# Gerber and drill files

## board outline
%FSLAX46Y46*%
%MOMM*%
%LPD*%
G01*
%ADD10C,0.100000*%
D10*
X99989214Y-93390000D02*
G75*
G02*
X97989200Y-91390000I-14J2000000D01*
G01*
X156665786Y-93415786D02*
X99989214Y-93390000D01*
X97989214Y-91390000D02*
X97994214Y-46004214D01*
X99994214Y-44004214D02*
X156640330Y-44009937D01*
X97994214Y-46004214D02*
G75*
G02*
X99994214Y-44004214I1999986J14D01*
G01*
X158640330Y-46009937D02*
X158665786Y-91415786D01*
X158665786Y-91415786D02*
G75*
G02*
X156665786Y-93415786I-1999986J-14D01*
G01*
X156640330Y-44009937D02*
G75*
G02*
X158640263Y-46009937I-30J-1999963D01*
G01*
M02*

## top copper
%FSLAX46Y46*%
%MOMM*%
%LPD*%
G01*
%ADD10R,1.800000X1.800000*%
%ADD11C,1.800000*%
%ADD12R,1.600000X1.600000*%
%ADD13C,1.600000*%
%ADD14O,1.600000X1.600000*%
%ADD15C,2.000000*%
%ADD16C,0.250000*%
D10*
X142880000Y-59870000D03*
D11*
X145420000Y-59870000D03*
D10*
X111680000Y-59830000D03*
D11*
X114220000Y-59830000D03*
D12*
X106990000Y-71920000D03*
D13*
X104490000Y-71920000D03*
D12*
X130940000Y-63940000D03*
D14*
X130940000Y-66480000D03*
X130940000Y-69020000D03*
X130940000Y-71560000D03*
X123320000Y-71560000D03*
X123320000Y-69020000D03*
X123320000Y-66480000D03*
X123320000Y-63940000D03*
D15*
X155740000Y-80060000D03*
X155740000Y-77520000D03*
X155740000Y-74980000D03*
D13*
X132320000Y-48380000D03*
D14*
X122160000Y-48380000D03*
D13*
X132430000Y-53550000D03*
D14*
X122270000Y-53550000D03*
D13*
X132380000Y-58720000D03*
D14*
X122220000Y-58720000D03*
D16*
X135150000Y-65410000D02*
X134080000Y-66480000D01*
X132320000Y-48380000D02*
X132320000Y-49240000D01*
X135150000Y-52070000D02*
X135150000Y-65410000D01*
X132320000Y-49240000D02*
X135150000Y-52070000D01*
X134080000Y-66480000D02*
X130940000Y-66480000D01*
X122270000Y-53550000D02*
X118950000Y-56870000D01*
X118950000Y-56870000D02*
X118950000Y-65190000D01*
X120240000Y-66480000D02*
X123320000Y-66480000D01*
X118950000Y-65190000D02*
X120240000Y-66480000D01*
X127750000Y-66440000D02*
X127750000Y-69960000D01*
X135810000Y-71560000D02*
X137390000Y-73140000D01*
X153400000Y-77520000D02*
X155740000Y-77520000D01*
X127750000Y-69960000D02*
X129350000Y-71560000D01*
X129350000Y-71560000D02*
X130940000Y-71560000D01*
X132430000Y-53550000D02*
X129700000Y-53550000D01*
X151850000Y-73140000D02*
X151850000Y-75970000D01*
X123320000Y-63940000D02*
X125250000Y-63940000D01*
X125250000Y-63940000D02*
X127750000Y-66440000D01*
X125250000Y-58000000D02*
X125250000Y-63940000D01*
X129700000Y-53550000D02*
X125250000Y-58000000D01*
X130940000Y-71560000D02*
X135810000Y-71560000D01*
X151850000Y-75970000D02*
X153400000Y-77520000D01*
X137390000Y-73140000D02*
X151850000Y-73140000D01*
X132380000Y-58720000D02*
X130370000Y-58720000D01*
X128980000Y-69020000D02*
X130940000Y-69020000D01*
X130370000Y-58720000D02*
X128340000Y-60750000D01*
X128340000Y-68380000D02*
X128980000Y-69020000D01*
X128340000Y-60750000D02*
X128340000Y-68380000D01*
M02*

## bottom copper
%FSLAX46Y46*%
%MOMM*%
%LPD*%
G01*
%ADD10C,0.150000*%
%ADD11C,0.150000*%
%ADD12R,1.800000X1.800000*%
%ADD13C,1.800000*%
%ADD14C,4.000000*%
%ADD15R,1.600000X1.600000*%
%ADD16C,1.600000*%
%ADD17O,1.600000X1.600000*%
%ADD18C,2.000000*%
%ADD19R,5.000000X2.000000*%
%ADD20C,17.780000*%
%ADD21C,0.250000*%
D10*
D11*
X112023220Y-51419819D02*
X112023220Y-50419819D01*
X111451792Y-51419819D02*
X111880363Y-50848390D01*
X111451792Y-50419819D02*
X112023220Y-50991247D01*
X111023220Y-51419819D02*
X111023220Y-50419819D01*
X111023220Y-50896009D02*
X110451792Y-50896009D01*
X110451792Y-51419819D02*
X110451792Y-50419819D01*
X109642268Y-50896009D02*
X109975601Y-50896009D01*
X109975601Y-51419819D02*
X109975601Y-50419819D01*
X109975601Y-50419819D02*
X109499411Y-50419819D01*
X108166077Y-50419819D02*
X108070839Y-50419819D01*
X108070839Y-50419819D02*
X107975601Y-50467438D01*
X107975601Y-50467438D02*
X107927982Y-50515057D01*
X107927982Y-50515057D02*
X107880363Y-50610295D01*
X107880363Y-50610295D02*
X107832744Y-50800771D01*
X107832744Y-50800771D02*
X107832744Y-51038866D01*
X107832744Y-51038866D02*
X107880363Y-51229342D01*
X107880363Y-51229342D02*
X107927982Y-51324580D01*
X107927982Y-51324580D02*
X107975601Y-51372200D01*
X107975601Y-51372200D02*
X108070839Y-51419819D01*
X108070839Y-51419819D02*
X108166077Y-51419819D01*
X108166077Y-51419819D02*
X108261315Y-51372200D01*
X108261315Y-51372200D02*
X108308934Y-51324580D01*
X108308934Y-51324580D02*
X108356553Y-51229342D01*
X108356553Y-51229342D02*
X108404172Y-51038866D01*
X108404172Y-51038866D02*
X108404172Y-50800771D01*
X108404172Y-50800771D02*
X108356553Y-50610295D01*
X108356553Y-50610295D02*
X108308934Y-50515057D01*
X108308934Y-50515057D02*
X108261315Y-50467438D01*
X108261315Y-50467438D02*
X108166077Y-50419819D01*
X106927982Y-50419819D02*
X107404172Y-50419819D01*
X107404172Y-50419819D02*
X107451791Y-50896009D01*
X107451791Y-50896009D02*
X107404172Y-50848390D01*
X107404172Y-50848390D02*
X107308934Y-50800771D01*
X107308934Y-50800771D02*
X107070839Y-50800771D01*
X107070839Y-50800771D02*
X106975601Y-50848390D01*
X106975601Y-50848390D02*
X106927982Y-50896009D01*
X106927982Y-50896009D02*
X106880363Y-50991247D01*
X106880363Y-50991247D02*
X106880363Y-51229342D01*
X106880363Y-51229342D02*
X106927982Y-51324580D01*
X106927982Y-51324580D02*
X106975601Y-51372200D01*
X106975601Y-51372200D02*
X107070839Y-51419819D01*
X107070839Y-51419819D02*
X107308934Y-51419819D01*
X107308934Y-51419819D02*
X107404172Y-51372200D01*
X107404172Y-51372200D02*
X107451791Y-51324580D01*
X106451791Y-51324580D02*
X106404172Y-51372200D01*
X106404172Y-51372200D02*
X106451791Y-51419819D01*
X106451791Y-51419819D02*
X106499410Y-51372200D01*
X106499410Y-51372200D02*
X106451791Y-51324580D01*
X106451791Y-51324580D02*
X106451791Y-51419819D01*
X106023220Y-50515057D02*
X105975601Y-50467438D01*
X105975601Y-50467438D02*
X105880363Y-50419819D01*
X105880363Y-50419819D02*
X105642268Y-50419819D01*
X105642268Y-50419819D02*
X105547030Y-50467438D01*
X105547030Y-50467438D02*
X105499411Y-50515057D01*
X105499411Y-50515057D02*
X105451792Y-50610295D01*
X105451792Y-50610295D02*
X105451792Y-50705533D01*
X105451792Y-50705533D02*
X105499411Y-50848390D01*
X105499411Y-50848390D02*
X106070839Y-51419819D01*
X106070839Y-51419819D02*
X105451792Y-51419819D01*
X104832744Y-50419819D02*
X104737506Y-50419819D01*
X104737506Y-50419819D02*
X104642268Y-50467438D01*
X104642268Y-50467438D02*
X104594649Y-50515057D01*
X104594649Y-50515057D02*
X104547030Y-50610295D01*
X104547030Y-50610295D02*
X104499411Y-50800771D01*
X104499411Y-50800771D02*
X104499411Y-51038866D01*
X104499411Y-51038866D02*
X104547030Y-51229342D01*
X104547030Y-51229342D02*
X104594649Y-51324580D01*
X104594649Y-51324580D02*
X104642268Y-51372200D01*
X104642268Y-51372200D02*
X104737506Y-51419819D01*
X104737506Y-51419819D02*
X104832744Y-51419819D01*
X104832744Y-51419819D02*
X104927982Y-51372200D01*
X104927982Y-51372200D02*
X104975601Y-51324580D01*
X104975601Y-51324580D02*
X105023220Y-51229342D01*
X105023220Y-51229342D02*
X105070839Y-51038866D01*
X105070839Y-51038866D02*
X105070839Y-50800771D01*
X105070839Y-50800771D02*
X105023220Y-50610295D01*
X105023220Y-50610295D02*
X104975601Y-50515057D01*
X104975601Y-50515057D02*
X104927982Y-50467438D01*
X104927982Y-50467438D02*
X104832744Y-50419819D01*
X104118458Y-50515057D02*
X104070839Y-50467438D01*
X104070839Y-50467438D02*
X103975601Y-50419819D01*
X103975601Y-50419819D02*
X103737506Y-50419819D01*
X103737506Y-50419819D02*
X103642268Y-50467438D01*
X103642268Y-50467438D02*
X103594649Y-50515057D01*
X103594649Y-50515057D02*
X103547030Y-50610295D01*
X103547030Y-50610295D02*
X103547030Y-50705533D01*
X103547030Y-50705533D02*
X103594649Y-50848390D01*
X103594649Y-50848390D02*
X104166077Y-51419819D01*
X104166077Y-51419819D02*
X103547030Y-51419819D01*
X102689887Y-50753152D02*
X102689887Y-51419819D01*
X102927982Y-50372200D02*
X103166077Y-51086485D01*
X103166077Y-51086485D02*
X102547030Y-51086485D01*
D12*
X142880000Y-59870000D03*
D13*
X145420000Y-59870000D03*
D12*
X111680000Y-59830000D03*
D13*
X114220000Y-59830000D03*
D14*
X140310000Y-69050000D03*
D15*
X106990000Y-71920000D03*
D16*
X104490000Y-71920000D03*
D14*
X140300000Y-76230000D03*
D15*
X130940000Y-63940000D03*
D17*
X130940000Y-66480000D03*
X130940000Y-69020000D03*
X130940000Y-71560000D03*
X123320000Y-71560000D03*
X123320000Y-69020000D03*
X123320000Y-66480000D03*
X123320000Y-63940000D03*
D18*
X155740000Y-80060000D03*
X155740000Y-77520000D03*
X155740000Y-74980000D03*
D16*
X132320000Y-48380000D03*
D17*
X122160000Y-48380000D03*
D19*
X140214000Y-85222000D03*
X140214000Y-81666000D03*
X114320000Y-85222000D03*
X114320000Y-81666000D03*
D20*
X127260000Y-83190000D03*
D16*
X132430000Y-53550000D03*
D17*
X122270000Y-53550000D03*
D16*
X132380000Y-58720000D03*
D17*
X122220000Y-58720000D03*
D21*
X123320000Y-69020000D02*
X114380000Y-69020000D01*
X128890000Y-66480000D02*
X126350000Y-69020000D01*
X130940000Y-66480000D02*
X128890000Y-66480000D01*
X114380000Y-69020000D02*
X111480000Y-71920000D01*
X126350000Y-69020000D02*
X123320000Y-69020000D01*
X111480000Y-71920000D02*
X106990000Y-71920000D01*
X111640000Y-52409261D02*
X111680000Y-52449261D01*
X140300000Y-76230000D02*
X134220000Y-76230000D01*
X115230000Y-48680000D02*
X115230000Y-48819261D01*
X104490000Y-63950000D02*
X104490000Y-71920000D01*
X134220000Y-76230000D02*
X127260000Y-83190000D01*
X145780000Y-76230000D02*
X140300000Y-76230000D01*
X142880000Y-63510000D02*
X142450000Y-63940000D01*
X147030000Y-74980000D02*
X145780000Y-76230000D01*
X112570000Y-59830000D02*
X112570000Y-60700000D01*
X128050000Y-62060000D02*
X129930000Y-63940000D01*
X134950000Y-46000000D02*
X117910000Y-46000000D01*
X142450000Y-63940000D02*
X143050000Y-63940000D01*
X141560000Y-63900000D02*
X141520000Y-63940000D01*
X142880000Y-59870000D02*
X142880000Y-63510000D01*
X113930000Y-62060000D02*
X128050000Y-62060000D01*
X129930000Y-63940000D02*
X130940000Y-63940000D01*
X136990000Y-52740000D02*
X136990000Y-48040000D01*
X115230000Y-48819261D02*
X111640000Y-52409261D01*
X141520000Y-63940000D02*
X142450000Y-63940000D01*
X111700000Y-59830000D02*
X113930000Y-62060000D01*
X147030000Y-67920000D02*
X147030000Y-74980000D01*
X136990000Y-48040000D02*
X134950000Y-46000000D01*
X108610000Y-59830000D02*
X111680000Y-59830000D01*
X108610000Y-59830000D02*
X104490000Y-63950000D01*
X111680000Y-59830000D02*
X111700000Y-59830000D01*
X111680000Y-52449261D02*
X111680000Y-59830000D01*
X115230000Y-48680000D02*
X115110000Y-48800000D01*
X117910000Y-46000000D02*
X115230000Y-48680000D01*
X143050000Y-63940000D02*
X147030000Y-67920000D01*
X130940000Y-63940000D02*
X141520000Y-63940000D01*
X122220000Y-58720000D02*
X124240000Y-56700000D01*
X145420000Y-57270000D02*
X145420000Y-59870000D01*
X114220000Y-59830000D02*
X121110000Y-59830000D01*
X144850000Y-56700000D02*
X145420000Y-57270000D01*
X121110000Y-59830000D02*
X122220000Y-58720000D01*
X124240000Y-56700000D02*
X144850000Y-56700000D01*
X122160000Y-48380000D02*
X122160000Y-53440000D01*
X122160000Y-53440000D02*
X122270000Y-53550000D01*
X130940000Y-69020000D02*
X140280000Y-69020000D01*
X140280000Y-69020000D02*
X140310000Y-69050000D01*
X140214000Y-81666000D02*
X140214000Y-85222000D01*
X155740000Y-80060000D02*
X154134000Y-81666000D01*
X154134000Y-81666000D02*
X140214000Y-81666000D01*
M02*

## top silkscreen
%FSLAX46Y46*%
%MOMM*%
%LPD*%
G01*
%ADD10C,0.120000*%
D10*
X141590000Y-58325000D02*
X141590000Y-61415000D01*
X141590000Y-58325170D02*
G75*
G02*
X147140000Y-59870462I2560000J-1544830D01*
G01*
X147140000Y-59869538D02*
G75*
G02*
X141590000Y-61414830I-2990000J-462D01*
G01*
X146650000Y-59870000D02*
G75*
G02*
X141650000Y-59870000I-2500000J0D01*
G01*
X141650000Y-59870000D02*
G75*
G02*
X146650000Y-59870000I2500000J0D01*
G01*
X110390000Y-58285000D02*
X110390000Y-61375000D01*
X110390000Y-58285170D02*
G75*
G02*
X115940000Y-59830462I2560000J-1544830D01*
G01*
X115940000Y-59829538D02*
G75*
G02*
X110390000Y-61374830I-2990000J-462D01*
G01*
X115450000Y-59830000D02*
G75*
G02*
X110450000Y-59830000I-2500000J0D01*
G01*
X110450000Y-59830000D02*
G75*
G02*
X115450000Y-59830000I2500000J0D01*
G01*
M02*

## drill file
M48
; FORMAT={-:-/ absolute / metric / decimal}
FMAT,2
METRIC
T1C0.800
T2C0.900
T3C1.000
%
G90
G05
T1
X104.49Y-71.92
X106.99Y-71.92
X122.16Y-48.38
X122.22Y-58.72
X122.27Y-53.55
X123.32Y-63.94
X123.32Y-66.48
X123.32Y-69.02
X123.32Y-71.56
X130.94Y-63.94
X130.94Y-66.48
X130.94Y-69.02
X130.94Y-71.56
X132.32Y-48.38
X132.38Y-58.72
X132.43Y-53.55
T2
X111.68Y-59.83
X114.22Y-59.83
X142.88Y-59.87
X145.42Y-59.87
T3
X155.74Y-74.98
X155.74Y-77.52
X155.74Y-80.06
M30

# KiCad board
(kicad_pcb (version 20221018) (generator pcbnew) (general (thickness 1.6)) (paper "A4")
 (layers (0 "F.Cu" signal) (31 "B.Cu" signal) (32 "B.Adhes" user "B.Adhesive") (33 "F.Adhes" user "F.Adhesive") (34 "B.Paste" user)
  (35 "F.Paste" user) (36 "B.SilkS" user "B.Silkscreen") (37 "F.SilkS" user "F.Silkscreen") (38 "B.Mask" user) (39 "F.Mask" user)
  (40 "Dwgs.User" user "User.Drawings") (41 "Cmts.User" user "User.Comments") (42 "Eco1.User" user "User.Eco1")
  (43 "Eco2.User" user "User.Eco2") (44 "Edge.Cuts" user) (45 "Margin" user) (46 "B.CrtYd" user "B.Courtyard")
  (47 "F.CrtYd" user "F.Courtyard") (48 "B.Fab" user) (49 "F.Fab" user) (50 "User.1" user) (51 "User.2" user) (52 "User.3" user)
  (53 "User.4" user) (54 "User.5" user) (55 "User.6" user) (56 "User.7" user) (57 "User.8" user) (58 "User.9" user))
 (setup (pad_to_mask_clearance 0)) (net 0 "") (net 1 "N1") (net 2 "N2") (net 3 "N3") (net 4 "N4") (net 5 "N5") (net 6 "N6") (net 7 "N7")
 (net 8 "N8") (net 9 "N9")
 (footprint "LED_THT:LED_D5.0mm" (layer "F.Cu") (at 142.88 59.87)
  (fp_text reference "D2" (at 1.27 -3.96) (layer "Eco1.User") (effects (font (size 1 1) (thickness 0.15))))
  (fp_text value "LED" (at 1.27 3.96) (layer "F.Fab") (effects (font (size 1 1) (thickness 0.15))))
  (fp_line (start -1.29 -1.545) (end -1.29 1.545) (stroke (width 0.12) (type solid)) (layer "F.SilkS"))
  (fp_arc (start -1.29 -1.54483) (mid 2.072002 -2.880433) (end 4.26 0.000462) (stroke (width 0.12) (type solid)) (layer "F.SilkS"))
  (fp_arc (start 4.26 -0.000462) (mid 2.072002 2.880433) (end -1.29 1.54483) (stroke (width 0.12) (type solid)) (layer "F.SilkS"))
  (fp_circle (center 1.27 0) (end 3.77 0) (stroke (width 0.12) (type solid)) (fill none) (layer "F.SilkS"))
  (pad "1" thru_hole rect (at 0 0) (size 1.8 1.8) (drill 0.9) (layers "*.Cu" "*.Mask") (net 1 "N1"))
  (pad "2" thru_hole circle (at 2.54 0) (size 1.8 1.8) (drill 0.9) (layers "*.Cu" "*.Mask") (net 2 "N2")))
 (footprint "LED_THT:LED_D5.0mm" (layer "F.Cu") (at 111.68 59.83)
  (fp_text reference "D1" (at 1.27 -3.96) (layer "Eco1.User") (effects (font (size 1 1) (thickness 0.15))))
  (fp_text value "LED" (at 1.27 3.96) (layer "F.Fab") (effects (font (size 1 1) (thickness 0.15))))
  (fp_line (start -1.29 -1.545) (end -1.29 1.545) (stroke (width 0.12) (type solid)) (layer "F.SilkS"))
  (fp_arc (start -1.29 -1.54483) (mid 2.072002 -2.880433) (end 4.26 0.000462) (stroke (width 0.12) (type solid)) (layer "F.SilkS"))
  (fp_arc (start 4.26 -0.000462) (mid 2.072002 2.880433) (end -1.29 1.54483) (stroke (width 0.12) (type solid)) (layer "F.SilkS"))
  (fp_circle (center 1.27 0) (end 3.77 0) (stroke (width 0.12) (type solid)) (fill none) (layer "F.SilkS"))
  (pad "1" thru_hole rect (at 0 0) (size 1.8 1.8) (drill 0.9) (layers "*.Cu" "*.Mask") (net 1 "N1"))
  (pad "2" thru_hole circle (at 2.54 0) (size 1.8 1.8) (drill 0.9) (layers "*.Cu" "*.Mask") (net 2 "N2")))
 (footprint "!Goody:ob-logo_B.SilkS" (layer "F.Cu") (at 151.17 67.66)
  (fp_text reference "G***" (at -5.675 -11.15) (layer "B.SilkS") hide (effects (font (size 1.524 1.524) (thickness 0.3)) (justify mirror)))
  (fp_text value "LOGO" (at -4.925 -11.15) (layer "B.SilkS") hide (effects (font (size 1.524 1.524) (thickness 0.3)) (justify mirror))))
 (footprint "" (layer "F.Cu") (at 140.31 69.05)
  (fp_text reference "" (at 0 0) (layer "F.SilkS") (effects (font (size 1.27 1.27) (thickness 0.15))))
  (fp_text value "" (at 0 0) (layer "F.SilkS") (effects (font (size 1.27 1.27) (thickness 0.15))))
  (pad "1" smd circle (at 0 0 180) (size 4 4) (layers "B.Cu" "B.Paste" "B.Mask") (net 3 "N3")))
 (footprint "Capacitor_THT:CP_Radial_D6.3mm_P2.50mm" (layer "B.Cu") (at 106.99 71.92 180)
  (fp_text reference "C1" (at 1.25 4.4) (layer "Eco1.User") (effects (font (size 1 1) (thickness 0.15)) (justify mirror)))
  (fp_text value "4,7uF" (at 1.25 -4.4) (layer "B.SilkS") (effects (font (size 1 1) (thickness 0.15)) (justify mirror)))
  (pad "1" thru_hole rect (at 0 0 180) (size 1.6 1.6) (drill 0.8) (layers "*.Cu" "*.Mask") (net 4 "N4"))
  (pad "2" thru_hole circle (at 2.5 0 180) (size 1.6 1.6) (drill 0.8) (layers "*.Cu" "*.Mask") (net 1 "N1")))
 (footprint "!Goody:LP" (layer "B.Cu") (at 140.3 76.23 180)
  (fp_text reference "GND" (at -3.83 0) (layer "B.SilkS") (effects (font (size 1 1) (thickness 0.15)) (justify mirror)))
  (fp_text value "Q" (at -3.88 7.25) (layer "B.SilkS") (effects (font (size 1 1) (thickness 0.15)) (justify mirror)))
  (pad "1" smd circle (at 0 0 180) (size 4 4) (layers "B.Cu" "B.Paste" "B.Mask") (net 1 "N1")))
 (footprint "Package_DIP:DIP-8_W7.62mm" (layer "B.Cu") (at 130.94 63.94 180)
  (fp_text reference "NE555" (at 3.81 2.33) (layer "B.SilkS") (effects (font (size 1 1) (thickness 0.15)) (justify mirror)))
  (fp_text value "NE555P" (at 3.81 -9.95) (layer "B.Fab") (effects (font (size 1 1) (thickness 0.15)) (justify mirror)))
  (pad "1" thru_hole rect (at 0 0 180) (size 1.6 1.6) (drill 0.8) (layers "*.Cu" "*.Mask") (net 1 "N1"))
  (pad "2" thru_hole oval (at 0 -2.54 180) (size 1.6 1.6) (drill 0.8) (layers "*.Cu" "*.Mask") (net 4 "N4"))
  (pad "3" thru_hole oval (at 0 -5.08 180) (size 1.6 1.6) (drill 0.8) (layers "*.Cu" "*.Mask") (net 3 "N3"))
  (pad "4" thru_hole oval (at 0 -7.62 180) (size 1.6 1.6) (drill 0.8) (layers "*.Cu" "*.Mask") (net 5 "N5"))
  (pad "5" thru_hole oval (at 7.62 -7.62 180) (size 1.6 1.6) (drill 0.8) (layers "*.Cu" "*.Mask") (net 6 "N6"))
  (pad "6" thru_hole oval (at 7.62 -5.08 180) (size 1.6 1.6) (drill 0.8) (layers "*.Cu" "*.Mask") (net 4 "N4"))
  (pad "7" thru_hole oval (at 7.62 -2.54 180) (size 1.6 1.6) (drill 0.8) (layers "*.Cu" "*.Mask") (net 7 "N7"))
  (pad "8" thru_hole oval (at 7.62 0 180) (size 1.6 1.6) (drill 0.8) (layers "*.Cu" "*.Mask") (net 5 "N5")))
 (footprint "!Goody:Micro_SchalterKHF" (layer "B.Cu") (at 155.74 80.06 90)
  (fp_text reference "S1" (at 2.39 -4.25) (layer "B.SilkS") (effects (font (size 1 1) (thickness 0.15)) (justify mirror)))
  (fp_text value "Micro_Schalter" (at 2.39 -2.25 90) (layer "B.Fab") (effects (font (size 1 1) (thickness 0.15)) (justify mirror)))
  (pad "1" thru_hole circle (at 0 0 90) (size 2 2) (drill 1) (layers "*.Cu" "*.Mask") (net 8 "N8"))
  (pad "2" thru_hole circle (at 2.54 0 90) (size 2 2) (drill 1) (layers "*.Cu" "*.Mask") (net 5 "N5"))
  (pad "3" thru_hole circle (at 5.08 0 90) (size 2 2) (drill 1) (layers "*.Cu" "*.Mask") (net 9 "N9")))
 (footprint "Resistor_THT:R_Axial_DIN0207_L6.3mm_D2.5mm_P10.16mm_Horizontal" (layer "B.Cu") (at 132.32 48.38 180)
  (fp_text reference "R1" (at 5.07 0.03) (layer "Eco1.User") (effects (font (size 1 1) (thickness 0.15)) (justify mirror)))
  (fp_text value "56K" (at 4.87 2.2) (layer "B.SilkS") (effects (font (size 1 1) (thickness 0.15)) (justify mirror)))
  (pad "1" thru_hole circle (at 0 0 180) (size 1.6 1.6) (drill 0.8) (layers "*.Cu" "*.Mask") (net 4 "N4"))
  (pad "2" thru_hole oval (at 10.16 0 180) (size 1.6 1.6) (drill 0.8) (layers "*.Cu" "*.Mask") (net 7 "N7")))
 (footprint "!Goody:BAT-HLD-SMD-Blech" (layer "B.Cu") (at 127.26 83.19 180)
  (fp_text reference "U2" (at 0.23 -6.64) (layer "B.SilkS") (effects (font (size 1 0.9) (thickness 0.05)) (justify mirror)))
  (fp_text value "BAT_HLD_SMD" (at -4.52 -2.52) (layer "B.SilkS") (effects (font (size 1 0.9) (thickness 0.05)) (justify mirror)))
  (pad "" smd rect (at -12.954 -2.032 180) (size 5 2) (layers "B.Cu" "B.Paste" "B.Mask") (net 8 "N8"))
  (pad "" smd rect (at -12.954 1.524 180) (size 5 2) (layers "B.Cu" "B.Paste" "B.Mask") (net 8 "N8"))
  (pad "1" smd rect (at 12.94 -2.032 180) (size 5 2) (layers "B.Cu" "B.Paste" "B.Mask"))
  (pad "1" smd rect (at 12.94 1.524 180) (size 5 2) (layers "B.Cu" "B.Paste" "B.Mask"))
  (pad "2" smd circle (at 0 0 180) (size 17.78 17.78) (layers "B.Cu" "B.Paste" "B.Mask") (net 1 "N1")))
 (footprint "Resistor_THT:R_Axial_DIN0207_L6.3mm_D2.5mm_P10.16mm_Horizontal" (layer "B.Cu") (at 132.43 53.55 180)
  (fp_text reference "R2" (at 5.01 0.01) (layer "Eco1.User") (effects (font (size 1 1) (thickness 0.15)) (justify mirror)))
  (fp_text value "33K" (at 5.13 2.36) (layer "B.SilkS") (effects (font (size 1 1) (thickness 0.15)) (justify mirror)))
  (pad "1" thru_hole circle (at 0 0 180) (size 1.6 1.6) (drill 0.8) (layers "*.Cu" "*.Mask") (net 5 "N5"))
  (pad "2" thru_hole oval (at 10.16 0 180) (size 1.6 1.6) (drill 0.8) (layers "*.Cu" "*.Mask") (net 7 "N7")))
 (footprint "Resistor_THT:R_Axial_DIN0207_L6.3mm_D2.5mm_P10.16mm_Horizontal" (layer "B.Cu") (at 132.38 58.72 180)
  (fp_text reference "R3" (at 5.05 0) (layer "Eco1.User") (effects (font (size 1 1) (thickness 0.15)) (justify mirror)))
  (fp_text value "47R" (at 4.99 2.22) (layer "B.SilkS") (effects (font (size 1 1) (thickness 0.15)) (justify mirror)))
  (pad "1" thru_hole circle (at 0 0 180) (size 1.6 1.6) (drill 0.8) (layers "*.Cu" "*.Mask") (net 3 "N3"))
  (pad "2" thru_hole oval (at 10.16 0 180) (size 1.6 1.6) (drill 0.8) (layers "*.Cu" "*.Mask") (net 2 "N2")))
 (gr_arc (start 99.989214 93.39) (mid 98.575 92.804214) (end 97.989214 91.39) (stroke (width 0.1) (type default)) (layer "Edge.Cuts"))
 (gr_line (start 156.665786 93.415786) (end 99.989214 93.39) (stroke (width 0.1) (type default)) (layer "Edge.Cuts"))
 (gr_line (start 97.989214 91.39) (end 97.994214 46.004214) (stroke (width 0.1) (type default)) (layer "Edge.Cuts"))
 (gr_line (start 99.994214 44.004214) (end 156.64033 44.009937) (stroke (width 0.1) (type default)) (layer "Edge.Cuts"))
 (gr_arc (start 97.994214 46.004214) (mid 98.58 44.59) (end 99.994214 44.004214) (stroke (width 0.1) (type default)) (layer "Edge.Cuts"))
 (gr_line (start 158.64033 46.009937) (end 158.665786 91.415786) (stroke (width 0.1) (type default)) (layer "Edge.Cuts"))
 (gr_arc (start 158.665786 91.415786) (mid 158.08 92.83) (end 156.665786 93.415786) (stroke (width 0.1) (type default)) (layer "Edge.Cuts"))
 (gr_arc (start 156.64033 44.009937) (mid 158.054544 44.595723) (end 158.64033 46.009937) (stroke (width 0.1) (type default))
  (layer "Edge.Cuts"))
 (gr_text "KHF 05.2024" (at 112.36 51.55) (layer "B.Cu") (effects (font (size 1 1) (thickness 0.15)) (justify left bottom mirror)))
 (segment (start 135.15 65.41) (end 134.08 66.48) (width 0.25) (layer "F.Cu") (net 4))
 (segment (start 132.32 48.38) (end 132.32 49.24) (width 0.25) (layer "F.Cu") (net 4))
 (segment (start 135.15 52.07) (end 135.15 65.41) (width 0.25) (layer "F.Cu") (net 4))
 (segment (start 132.32 49.24) (end 135.15 52.07) (width 0.25) (layer "F.Cu") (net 4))
 (segment (start 134.08 66.48) (end 130.94 66.48) (width 0.25) (layer "F.Cu") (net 4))
 (segment (start 123.32 69.02) (end 114.38 69.02) (width 0.25) (layer "B.Cu") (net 4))
 (segment (start 128.89 66.48) (end 126.35 69.02) (width 0.25) (layer "B.Cu") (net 4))
 (segment (start 130.94 66.48) (end 128.89 66.48) (width 0.25) (layer "B.Cu") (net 4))
 (segment (start 114.38 69.02) (end 111.48 71.92) (width 0.25) (layer "B.Cu") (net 4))
 (segment (start 126.35 69.02) (end 123.32 69.02) (width 0.25) (layer "B.Cu") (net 4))
 (segment (start 111.48 71.92) (end 106.99 71.92) (width 0.25) (layer "B.Cu") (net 4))
 (segment (start 111.64 52.409261) (end 111.68 52.449261) (width 0.25) (layer "B.Cu") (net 1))
 (segment (start 140.3 76.23) (end 134.22 76.23) (width 0.25) (layer "B.Cu") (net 1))
 (segment (start 115.23 48.68) (end 115.23 48.819261) (width 0.25) (layer "B.Cu") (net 1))
 (segment (start 104.49 63.95) (end 104.49 71.92) (width 0.25) (layer "B.Cu") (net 1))
 (segment (start 134.22 76.23) (end 127.26 83.19) (width 0.25) (layer "B.Cu") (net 1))
 (segment (start 145.78 76.23) (end 140.3 76.23) (width 0.25) (layer "B.Cu") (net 1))
 (segment (start 142.88 63.51) (end 142.45 63.94) (width 0.25) (layer "B.Cu") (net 1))
 (segment (start 147.03 74.98) (end 145.78 76.23) (width 0.25) (layer "B.Cu") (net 1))
 (segment (start 112.57 59.83) (end 112.57 60.7) (width 0.25) (layer "B.Cu") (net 1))
 (segment (start 128.05 62.06) (end 129.93 63.94) (width 0.25) (layer "B.Cu") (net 1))
 (segment (start 134.95 46) (end 117.91 46) (width 0.25) (layer "B.Cu") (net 1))
 (segment (start 142.45 63.94) (end 143.05 63.94) (width 0.25) (layer "B.Cu") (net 1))
 (segment (start 141.56 63.9) (end 141.52 63.94) (width 0.25) (layer "B.Cu") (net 1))
 (segment (start 142.88 59.87) (end 142.88 63.51) (width 0.25) (layer "B.Cu") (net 1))
 (segment (start 113.93 62.06) (end 128.05 62.06) (width 0.25) (layer "B.Cu") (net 1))
 (segment (start 129.93 63.94) (end 130.94 63.94) (width 0.25) (layer "B.Cu") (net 1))
 (segment (start 136.99 52.74) (end 136.99 48.04) (width 0.25) (layer "B.Cu") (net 1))
 (segment (start 115.23 48.819261) (end 111.64 52.409261) (width 0.25) (layer "B.Cu") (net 1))
 (segment (start 141.52 63.94) (end 142.45 63.94) (width 0.25) (layer "B.Cu") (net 1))
 (segment (start 111.7 59.83) (end 113.93 62.06) (width 0.25) (layer "B.Cu") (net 1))
 (segment (start 147.03 67.92) (end 147.03 74.98) (width 0.25) (layer "B.Cu") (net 1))
 (segment (start 136.99 48.04) (end 134.95 46) (width 0.25) (layer "B.Cu") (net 1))
 (segment (start 108.61 59.83) (end 111.68 59.83) (width 0.25) (layer "B.Cu") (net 1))
 (segment (start 108.61 59.83) (end 104.49 63.95) (width 0.25) (layer "B.Cu") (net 1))
 (segment (start 111.68 59.83) (end 111.7 59.83) (width 0.25) (layer "B.Cu") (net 1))
 (segment (start 111.68 52.449261) (end 111.68 59.83) (width 0.25) (layer "B.Cu") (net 1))
 (segment (start 115.23 48.68) (end 115.11 48.8) (width 0.25) (layer "B.Cu") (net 1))
 (segment (start 117.91 46) (end 115.23 48.68) (width 0.25) (layer "B.Cu") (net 1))
 (segment (start 143.05 63.94) (end 147.03 67.92) (width 0.25) (layer "B.Cu") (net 1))
 (segment (start 130.94 63.94) (end 141.52 63.94) (width 0.25) (layer "B.Cu") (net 1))
 (segment (start 122.22 58.72) (end 124.24 56.7) (width 0.25) (layer "B.Cu") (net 2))
 (segment (start 145.42 57.27) (end 145.42 59.87) (width 0.25) (layer "B.Cu") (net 2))
 (segment (start 114.22 59.83) (end 121.11 59.83) (width 0.25) (layer "B.Cu") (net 2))
 (segment (start 144.85 56.7) (end 145.42 57.27) (width 0.25) (layer "B.Cu") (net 2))
 (segment (start 121.11 59.83) (end 122.22 58.72) (width 0.25) (layer "B.Cu") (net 2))
 (segment (start 124.24 56.7) (end 144.85 56.7) (width 0.25) (layer "B.Cu") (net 2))
 (segment (start 122.27 53.55) (end 118.95 56.87) (width 0.25) (layer "F.Cu") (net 7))
 (segment (start 118.95 56.87) (end 118.95 65.19) (width 0.25) (layer "F.Cu") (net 7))
 (segment (start 120.24 66.48) (end 123.32 66.48) (width 0.25) (layer "F.Cu") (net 7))
 (segment (start 118.95 65.19) (end 120.24 66.48) (width 0.25) (layer "F.Cu") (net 7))
 (segment (start 122.16 48.38) (end 122.16 53.44) (width 0.25) (layer "B.Cu") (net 7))
 (segment (start 122.16 53.44) (end 122.27 53.55) (width 0.25) (layer "B.Cu") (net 7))
 (segment (start 127.75 66.44) (end 127.75 69.96) (width 0.25) (layer "F.Cu") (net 5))
 (segment (start 135.81 71.56) (end 137.39 73.14) (width 0.25) (layer "F.Cu") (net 5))
 (segment (start 153.4 77.52) (end 155.74 77.52) (width 0.25) (layer "F.Cu") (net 5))
 (segment (start 127.75 69.96) (end 129.35 71.56) (width 0.25) (layer "F.Cu") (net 5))
 (segment (start 129.35 71.56) (end 130.94 71.56) (width 0.25) (layer "F.Cu") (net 5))
 (segment (start 132.43 53.55) (end 129.7 53.55) (width 0.25) (layer "F.Cu") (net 5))
 (segment (start 151.85 73.14) (end 151.85 75.97) (width 0.25) (layer "F.Cu") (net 5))
 (segment (start 123.32 63.94) (end 125.25 63.94) (width 0.25) (layer "F.Cu") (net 5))
 (segment (start 125.25 63.94) (end 127.75 66.44) (width 0.25) (layer "F.Cu") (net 5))
 (segment (start 125.25 58) (end 125.25 63.94) (width 0.25) (layer "F.Cu") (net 5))
 (segment (start 129.7 53.55) (end 125.25 58) (width 0.25) (layer "F.Cu") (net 5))
 (segment (start 130.94 71.56) (end 135.81 71.56) (width 0.25) (layer "F.Cu") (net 5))
 (segment (start 151.85 75.97) (end 153.4 77.52) (width 0.25) (layer "F.Cu") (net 5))
 (segment (start 137.39 73.14) (end 151.85 73.14) (width 0.25) (layer "F.Cu") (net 5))
 (segment (start 132.38 58.72) (end 130.37 58.72) (width 0.25) (layer "F.Cu") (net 3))
 (segment (start 128.98 69.02) (end 130.94 69.02) (width 0.25) (layer "F.Cu") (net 3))
 (segment (start 130.37 58.72) (end 128.34 60.75) (width 0.25) (layer "F.Cu") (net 3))
 (segment (start 128.34 68.38) (end 128.98 69.02) (width 0.25) (layer "F.Cu") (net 3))
 (segment (start 128.34 60.75) (end 128.34 68.38) (width 0.25) (layer "F.Cu") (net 3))
 (segment (start 130.94 69.02) (end 140.28 69.02) (width 0.25) (layer "B.Cu") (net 3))
 (segment (start 140.28 69.02) (end 140.31 69.05) (width 0.25) (layer "B.Cu") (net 3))
 (segment (start 140.214 81.666) (end 140.214 85.222) (width 0.25) (layer "B.Cu") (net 8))
 (segment (start 155.74 80.06) (end 154.134 81.666) (width 0.25) (layer "B.Cu") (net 8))
 (segment (start 154.134 81.666) (end 140.214 81.666) (width 0.25) (layer "B.Cu") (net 8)))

